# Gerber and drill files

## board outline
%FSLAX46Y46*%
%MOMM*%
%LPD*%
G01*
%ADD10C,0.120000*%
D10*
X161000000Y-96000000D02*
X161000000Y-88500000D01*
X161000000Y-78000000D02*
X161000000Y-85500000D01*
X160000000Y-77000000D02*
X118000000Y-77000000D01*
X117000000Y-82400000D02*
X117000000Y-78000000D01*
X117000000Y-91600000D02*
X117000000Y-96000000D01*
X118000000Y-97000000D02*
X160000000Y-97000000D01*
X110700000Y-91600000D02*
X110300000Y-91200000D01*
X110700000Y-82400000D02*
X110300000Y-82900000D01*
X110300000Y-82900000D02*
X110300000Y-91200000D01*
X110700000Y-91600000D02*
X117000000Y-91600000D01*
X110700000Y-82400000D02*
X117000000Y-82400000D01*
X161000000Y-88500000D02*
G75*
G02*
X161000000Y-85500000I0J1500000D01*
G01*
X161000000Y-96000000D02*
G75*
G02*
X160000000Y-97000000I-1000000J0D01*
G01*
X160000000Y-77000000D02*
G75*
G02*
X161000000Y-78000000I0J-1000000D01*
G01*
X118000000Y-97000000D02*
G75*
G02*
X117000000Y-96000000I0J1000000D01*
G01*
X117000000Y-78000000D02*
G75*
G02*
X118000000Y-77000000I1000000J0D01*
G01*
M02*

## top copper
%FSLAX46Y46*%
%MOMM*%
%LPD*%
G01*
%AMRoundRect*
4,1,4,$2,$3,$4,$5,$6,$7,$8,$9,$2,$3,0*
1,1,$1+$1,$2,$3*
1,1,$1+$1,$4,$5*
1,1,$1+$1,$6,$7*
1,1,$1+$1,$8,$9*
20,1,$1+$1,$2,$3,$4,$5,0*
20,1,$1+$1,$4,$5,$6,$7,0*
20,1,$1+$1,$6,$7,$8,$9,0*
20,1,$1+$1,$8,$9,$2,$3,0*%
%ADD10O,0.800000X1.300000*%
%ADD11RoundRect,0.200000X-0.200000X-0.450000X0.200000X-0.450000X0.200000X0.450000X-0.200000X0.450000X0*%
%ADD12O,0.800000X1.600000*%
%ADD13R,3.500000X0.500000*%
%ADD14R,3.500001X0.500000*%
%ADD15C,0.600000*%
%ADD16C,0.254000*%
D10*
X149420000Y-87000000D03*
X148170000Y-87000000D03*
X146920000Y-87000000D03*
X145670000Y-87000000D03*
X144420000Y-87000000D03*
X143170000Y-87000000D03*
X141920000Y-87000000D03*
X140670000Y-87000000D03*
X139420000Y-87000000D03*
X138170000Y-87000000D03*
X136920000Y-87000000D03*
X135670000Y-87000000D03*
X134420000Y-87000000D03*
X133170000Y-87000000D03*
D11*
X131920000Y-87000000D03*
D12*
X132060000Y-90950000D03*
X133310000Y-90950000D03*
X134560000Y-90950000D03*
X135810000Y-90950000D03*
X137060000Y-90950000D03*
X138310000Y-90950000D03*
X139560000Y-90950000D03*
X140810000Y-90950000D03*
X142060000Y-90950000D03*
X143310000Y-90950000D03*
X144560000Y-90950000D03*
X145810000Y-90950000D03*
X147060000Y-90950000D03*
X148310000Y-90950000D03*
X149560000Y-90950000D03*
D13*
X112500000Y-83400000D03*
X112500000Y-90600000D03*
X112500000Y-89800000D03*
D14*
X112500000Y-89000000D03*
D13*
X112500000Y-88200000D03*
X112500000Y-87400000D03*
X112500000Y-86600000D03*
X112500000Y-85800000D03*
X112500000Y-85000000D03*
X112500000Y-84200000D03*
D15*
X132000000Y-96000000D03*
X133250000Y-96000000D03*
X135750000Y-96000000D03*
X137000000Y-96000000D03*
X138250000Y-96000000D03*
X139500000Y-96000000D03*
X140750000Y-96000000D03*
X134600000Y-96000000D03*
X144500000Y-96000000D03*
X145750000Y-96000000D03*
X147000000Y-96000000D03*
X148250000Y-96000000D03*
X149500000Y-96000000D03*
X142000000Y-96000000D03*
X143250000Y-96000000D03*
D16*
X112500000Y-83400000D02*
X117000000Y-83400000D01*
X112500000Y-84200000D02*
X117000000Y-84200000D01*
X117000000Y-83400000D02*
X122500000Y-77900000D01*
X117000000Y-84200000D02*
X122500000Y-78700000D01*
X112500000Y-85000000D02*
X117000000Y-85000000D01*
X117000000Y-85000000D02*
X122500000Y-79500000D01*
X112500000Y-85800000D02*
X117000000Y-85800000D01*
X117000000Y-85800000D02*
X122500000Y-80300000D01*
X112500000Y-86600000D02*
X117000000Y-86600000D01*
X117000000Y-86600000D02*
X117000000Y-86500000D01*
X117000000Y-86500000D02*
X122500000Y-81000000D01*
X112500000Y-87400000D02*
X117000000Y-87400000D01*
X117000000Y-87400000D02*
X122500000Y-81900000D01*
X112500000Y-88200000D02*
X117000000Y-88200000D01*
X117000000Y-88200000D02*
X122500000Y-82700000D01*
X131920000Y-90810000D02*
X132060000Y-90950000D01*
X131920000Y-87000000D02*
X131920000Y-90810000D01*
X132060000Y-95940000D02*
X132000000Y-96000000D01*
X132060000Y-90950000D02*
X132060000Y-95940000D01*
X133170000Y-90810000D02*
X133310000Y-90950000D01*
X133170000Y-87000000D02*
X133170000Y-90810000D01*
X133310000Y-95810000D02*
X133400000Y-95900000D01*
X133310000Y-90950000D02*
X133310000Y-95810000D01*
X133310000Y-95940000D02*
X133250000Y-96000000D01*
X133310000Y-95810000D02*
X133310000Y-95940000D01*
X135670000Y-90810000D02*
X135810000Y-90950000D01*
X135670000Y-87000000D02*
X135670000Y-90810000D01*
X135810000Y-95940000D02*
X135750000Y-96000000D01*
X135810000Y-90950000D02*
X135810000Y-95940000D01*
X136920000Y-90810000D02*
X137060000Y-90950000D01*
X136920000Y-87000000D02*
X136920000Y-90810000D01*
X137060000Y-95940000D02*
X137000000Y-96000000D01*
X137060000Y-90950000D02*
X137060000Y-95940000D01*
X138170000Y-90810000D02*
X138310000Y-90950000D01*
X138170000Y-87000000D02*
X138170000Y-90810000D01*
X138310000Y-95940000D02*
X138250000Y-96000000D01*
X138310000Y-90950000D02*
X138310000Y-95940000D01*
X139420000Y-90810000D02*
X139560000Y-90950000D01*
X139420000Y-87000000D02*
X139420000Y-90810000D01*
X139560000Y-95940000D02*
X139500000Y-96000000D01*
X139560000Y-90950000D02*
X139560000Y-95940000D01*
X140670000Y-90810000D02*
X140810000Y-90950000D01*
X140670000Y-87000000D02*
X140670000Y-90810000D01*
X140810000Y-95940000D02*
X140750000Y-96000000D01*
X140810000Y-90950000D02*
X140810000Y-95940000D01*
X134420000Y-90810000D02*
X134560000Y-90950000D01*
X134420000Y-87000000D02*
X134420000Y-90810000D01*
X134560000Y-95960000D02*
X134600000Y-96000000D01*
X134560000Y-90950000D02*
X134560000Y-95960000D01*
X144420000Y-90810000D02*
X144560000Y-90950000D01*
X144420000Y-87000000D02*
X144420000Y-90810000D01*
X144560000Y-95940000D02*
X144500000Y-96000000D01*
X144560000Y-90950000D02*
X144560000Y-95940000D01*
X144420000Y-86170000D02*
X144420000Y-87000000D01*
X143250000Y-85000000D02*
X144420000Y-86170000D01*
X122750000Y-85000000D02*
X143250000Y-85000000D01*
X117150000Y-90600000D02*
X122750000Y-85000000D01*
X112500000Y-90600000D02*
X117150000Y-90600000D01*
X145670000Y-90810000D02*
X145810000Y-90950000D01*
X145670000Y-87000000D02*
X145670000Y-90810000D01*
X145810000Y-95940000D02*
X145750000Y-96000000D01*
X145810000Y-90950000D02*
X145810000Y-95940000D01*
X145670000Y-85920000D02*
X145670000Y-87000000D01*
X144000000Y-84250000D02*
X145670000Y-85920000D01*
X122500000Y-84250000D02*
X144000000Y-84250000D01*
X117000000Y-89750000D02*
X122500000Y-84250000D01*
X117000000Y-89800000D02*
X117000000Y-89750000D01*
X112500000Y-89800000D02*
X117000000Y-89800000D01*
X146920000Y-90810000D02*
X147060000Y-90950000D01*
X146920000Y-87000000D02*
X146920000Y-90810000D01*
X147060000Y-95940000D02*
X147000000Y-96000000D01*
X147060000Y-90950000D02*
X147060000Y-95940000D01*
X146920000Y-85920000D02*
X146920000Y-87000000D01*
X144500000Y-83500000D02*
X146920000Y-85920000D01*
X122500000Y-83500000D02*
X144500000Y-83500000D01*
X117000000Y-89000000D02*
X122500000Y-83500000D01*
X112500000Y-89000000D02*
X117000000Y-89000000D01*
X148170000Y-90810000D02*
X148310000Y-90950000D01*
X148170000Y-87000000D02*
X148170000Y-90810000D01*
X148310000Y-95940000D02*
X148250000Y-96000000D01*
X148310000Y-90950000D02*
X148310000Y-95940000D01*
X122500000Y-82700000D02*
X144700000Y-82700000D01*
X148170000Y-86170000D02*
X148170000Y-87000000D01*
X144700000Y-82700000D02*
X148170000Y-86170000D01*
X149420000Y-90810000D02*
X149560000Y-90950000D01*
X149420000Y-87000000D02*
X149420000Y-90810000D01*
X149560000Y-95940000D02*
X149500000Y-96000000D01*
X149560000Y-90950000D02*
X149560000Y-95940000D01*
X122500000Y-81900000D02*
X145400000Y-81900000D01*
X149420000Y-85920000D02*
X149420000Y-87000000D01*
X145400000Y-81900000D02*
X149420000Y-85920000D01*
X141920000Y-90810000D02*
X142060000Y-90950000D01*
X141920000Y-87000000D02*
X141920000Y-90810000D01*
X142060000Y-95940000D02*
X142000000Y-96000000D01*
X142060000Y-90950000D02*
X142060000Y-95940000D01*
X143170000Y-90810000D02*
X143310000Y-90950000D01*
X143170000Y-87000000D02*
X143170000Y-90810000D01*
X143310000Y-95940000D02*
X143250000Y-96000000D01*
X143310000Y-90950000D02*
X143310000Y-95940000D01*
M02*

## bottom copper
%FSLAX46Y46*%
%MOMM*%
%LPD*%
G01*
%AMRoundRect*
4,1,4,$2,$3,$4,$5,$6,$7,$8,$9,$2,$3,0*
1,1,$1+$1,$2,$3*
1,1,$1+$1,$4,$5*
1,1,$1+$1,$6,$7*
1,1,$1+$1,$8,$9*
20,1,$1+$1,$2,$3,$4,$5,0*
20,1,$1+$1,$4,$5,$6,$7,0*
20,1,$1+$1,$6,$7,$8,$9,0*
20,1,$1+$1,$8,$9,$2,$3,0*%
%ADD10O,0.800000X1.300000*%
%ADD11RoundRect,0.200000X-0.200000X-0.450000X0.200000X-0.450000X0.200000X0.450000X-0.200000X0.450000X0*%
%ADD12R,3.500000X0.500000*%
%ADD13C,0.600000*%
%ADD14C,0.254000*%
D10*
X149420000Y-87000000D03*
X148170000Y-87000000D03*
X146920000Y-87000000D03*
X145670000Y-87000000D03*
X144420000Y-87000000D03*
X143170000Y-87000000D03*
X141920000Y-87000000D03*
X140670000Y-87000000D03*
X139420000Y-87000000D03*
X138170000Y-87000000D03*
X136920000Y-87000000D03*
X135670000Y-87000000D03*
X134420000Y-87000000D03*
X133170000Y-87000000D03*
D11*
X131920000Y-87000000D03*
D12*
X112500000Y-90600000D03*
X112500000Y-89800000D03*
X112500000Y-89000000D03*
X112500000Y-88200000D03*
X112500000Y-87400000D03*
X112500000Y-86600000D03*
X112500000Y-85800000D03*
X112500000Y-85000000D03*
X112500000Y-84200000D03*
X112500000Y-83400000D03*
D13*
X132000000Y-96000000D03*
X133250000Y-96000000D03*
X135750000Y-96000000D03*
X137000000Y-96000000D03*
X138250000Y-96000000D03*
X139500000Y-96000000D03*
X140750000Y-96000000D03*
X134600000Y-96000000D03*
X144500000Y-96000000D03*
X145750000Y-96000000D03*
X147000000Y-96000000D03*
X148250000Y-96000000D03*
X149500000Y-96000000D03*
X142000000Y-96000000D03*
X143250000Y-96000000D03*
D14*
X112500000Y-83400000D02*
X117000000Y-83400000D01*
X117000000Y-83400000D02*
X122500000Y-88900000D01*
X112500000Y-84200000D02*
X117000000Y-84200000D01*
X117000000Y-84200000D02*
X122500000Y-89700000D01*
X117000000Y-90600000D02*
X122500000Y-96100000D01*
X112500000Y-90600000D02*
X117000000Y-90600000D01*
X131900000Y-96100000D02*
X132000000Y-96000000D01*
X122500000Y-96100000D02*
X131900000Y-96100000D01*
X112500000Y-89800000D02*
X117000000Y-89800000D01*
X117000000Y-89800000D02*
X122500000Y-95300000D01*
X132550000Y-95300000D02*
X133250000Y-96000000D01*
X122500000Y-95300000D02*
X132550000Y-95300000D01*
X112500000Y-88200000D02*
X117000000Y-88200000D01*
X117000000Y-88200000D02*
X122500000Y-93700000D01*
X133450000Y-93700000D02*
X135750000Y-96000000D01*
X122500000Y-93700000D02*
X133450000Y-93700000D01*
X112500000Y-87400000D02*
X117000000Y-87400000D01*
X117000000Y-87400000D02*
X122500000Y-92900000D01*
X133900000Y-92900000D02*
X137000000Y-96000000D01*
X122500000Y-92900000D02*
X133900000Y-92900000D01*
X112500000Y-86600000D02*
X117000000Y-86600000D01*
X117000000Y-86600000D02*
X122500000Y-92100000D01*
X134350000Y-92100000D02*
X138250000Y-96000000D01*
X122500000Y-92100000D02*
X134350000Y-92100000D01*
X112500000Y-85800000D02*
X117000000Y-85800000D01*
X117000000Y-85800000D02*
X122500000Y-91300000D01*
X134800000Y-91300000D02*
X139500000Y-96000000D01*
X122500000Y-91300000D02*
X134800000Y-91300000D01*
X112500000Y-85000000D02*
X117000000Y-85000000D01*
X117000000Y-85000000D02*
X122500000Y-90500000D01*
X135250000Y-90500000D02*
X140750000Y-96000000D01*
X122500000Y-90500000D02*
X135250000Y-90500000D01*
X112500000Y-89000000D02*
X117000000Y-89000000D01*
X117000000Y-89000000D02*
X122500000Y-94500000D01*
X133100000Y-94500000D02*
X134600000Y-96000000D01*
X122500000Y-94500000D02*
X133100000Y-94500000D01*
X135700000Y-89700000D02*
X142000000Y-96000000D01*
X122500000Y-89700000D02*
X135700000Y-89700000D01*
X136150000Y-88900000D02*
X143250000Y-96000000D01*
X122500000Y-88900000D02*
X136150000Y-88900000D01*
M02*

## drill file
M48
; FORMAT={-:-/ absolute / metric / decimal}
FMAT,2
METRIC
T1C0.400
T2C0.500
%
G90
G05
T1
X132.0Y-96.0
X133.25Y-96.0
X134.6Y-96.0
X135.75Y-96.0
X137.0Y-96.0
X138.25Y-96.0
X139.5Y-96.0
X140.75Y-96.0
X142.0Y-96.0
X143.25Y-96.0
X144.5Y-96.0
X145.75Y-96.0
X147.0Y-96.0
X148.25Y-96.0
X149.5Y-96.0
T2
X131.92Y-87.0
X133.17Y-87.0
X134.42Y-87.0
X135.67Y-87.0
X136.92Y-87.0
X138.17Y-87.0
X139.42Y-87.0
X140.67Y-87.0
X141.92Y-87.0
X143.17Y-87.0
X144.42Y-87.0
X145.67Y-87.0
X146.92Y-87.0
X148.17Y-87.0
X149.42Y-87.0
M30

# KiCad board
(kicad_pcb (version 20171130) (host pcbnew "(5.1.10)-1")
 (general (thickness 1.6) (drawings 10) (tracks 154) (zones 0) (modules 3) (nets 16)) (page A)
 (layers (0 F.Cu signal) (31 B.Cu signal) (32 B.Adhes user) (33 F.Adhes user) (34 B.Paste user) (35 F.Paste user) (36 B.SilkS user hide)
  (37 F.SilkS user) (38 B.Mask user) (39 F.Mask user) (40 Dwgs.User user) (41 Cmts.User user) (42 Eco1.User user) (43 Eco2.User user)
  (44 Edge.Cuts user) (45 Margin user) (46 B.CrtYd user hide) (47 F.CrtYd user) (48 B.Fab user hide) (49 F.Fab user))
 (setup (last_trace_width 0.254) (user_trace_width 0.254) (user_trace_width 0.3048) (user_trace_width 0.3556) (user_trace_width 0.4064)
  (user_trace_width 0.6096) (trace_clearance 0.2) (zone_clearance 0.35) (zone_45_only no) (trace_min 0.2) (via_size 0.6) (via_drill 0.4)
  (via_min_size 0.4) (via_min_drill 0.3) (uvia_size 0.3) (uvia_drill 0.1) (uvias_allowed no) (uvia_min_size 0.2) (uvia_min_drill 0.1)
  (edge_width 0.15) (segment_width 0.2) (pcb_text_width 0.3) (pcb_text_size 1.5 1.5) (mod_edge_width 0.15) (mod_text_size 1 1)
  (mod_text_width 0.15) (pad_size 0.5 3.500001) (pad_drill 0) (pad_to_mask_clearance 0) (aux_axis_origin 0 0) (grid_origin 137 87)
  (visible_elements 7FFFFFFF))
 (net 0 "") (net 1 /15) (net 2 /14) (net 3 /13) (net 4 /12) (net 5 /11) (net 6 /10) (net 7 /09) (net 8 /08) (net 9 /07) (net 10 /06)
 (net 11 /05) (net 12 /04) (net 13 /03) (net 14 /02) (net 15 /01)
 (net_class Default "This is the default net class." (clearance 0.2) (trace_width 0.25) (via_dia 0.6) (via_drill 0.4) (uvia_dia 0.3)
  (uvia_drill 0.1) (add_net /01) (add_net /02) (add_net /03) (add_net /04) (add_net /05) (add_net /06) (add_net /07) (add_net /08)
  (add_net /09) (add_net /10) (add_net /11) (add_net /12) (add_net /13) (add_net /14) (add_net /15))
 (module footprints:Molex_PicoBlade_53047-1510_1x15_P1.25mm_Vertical (layer F.Cu) (at 131.92 87)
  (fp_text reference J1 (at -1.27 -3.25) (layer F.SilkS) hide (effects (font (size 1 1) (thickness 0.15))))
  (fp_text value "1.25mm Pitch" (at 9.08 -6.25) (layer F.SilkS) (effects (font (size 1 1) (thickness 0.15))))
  (pad 15 thru_hole oval (at 17.5 0) (size 0.8 1.3) (drill 0.5) (layers *.Cu *.Mask) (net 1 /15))
  (pad 14 thru_hole oval (at 16.25 0) (size 0.8 1.3) (drill 0.5) (layers *.Cu *.Mask) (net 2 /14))
  (pad 13 thru_hole oval (at 15 0) (size 0.8 1.3) (drill 0.5) (layers *.Cu *.Mask) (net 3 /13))
  (pad 12 thru_hole oval (at 13.75 0) (size 0.8 1.3) (drill 0.5) (layers *.Cu *.Mask) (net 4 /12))
  (pad 11 thru_hole oval (at 12.5 0) (size 0.8 1.3) (drill 0.5) (layers *.Cu *.Mask) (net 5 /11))
  (pad 10 thru_hole oval (at 11.25 0) (size 0.8 1.3) (drill 0.5) (layers *.Cu *.Mask) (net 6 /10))
  (pad 9 thru_hole oval (at 10 0) (size 0.8 1.3) (drill 0.5) (layers *.Cu *.Mask) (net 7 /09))
  (pad 8 thru_hole oval (at 8.75 0) (size 0.8 1.3) (drill 0.5) (layers *.Cu *.Mask) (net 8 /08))
  (pad 7 thru_hole oval (at 7.5 0) (size 0.8 1.3) (drill 0.5) (layers *.Cu *.Mask) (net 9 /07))
  (pad 6 thru_hole oval (at 6.25 0) (size 0.8 1.3) (drill 0.5) (layers *.Cu *.Mask) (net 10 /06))
  (pad 5 thru_hole oval (at 5 0) (size 0.8 1.3) (drill 0.5) (layers *.Cu *.Mask) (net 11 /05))
  (pad 4 thru_hole oval (at 3.75 0) (size 0.8 1.3) (drill 0.5) (layers *.Cu *.Mask) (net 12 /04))
  (pad 3 thru_hole oval (at 2.5 0) (size 0.8 1.3) (drill 0.5) (layers *.Cu *.Mask) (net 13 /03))
  (pad 2 thru_hole oval (at 1.25 0) (size 0.8 1.3) (drill 0.5) (layers *.Cu *.Mask) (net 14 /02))
  (pad 1 thru_hole roundrect (at 0 0) (size 0.8 1.3) (drill 0.5) (layers *.Cu *.Mask) (roundrect_rratio 0.25) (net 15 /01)))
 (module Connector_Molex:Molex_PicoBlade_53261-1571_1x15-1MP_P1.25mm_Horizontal (layer F.Cu) (at 140.81 93.35)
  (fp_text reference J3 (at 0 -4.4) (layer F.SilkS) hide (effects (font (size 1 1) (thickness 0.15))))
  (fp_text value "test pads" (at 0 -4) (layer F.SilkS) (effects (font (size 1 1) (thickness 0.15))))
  (pad 1 smd oval (at -8.75 -2.4) (size 0.8 1.6) (layers F.Cu F.Paste F.Mask) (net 15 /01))
  (pad 2 smd oval (at -7.5 -2.4) (size 0.8 1.6) (layers F.Cu F.Paste F.Mask) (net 14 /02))
  (pad 3 smd oval (at -6.25 -2.4) (size 0.8 1.6) (layers F.Cu F.Paste F.Mask) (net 13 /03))
  (pad 4 smd oval (at -5 -2.4) (size 0.8 1.6) (layers F.Cu F.Paste F.Mask) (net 12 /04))
  (pad 5 smd oval (at -3.75 -2.4) (size 0.8 1.6) (layers F.Cu F.Paste F.Mask) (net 11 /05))
  (pad 6 smd oval (at -2.5 -2.4) (size 0.8 1.6) (layers F.Cu F.Paste F.Mask) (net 10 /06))
  (pad 7 smd oval (at -1.25 -2.4) (size 0.8 1.6) (layers F.Cu F.Paste F.Mask) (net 9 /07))
  (pad 8 smd oval (at 0 -2.4) (size 0.8 1.6) (layers F.Cu F.Paste F.Mask) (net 8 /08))
  (pad 9 smd oval (at 1.25 -2.4) (size 0.8 1.6) (layers F.Cu F.Paste F.Mask) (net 7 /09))
  (pad 10 smd oval (at 2.5 -2.4) (size 0.8 1.6) (layers F.Cu F.Paste F.Mask) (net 6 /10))
  (pad 11 smd oval (at 3.75 -2.4) (size 0.8 1.6) (layers F.Cu F.Paste F.Mask) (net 5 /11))
  (pad 12 smd oval (at 5 -2.4) (size 0.8 1.6) (layers F.Cu F.Paste F.Mask) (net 4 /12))
  (pad 13 smd oval (at 6.25 -2.4) (size 0.8 1.6) (layers F.Cu F.Paste F.Mask) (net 3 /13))
  (pad 14 smd oval (at 7.5 -2.4) (size 0.8 1.6) (layers F.Cu F.Paste F.Mask) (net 2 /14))
  (pad 15 smd oval (at 8.75 -2.4) (size 0.8 1.6) (layers F.Cu F.Paste F.Mask) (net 1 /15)))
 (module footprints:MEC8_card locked (layer F.Cu) (at 112.5 87 90)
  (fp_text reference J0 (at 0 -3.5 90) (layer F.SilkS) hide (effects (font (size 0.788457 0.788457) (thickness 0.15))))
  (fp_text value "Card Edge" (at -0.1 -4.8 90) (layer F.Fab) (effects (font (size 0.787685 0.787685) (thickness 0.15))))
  (fp_line (start -9 48.5) (end -1.5 48.5) (layer Edge.Cuts) (width 0.12))
  (fp_line (start 9 48.5) (end 1.5 48.5) (layer Edge.Cuts) (width 0.12))
  (fp_line (start 10 47.5) (end 10 5.5) (layer Edge.Cuts) (width 0.12))
  (fp_line (start 4.6 4.5) (end 9 4.5) (layer Edge.Cuts) (width 0.12))
  (fp_line (start -4.6 4.5) (end -9 4.5) (layer Edge.Cuts) (width 0.12))
  (fp_line (start -10 5.5) (end -10 47.5) (layer Edge.Cuts) (width 0.12))
  (fp_line (start -4.6 -1.8) (end -4.2 -2.2) (layer Edge.Cuts) (width 0.12))
  (fp_line (start 4.6 -1.8) (end 4.1 -2.2) (layer Edge.Cuts) (width 0.12))
  (fp_line (start 4.1 -2.2) (end -4.2 -2.2) (layer Edge.Cuts) (width 0.12))
  (fp_line (start -4.6 -1.8) (end -4.6 4.5) (layer Edge.Cuts) (width 0.12))
  (fp_line (start 4.6 -1.8) (end 4.6 4.5) (layer Edge.Cuts) (width 0.12))
  (fp_arc (start 0 48.5) (end 1.5 48.5) (angle -180) (layer Edge.Cuts) (width 0.12))
  (fp_arc (start -9 47.5) (end -10 47.5) (angle -90) (layer Edge.Cuts) (width 0.12))
  (fp_arc (start 9 47.5) (end 9 48.5) (angle -90) (layer Edge.Cuts) (width 0.12))
  (fp_arc (start -9 5.5) (end -9 4.5) (angle -90) (layer Edge.Cuts) (width 0.12))
  (fp_arc (start 9 5.5) (end 10 5.5) (angle -90) (layer Edge.Cuts) (width 0.12))
  (pad 20 smd rect (at 3.6 0 90) (size 0.5 3.5) (layers F.Cu F.Paste F.Mask))
  (pad 11 smd rect (at -3.6 0 90) (size 0.5 3.5) (layers F.Cu F.Paste F.Mask) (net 5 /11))
  (pad 12 smd rect (at -2.8 0 90) (size 0.5 3.5) (layers F.Cu F.Paste F.Mask) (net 4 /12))
  (pad 13 smd rect (at -2 0 90) (size 0.5 3.500001) (layers F.Cu F.Paste F.Mask) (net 3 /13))
  (pad 14 smd rect (at -1.2 0 90) (size 0.5 3.5) (layers F.Cu F.Paste F.Mask) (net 2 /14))
  (pad 15 smd rect (at -0.4 0 90) (size 0.5 3.5) (layers F.Cu F.Paste F.Mask) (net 1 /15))
  (pad 16 smd rect (at 0.4 0 90) (size 0.5 3.5) (layers F.Cu F.Paste F.Mask))
  (pad 17 smd rect (at 1.2 0 90) (size 0.5 3.5) (layers F.Cu F.Paste F.Mask))
  (pad 18 smd rect (at 2 0 90) (size 0.5 3.5) (layers F.Cu F.Paste F.Mask))
  (pad 19 smd rect (at 2.8 0 90) (size 0.5 3.5) (layers F.Cu F.Paste F.Mask))
  (pad 1 smd rect (at -3.6 0 90) (size 0.5 3.5) (layers B.Cu B.Paste B.Mask) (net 15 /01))
  (pad 2 smd rect (at -2.8 0 90) (size 0.5 3.5) (layers B.Cu B.Paste B.Mask) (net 14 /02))
  (pad 3 smd rect (at -2 0 90) (size 0.5 3.5) (layers B.Cu B.Paste B.Mask) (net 13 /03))
  (pad 4 smd rect (at -1.2 0 90) (size 0.5 3.5) (layers B.Cu B.Paste B.Mask) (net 12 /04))
  (pad 5 smd rect (at -0.4 0 90) (size 0.5 3.5) (layers B.Cu B.Paste B.Mask) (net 11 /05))
  (pad 6 smd rect (at 0.4 0 90) (size 0.5 3.5) (layers B.Cu B.Paste B.Mask) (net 10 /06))
  (pad 7 smd rect (at 1.2 0 90) (size 0.5 3.5) (layers B.Cu B.Paste B.Mask) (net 9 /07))
  (pad 8 smd rect (at 2 0 90) (size 0.5 3.5) (layers B.Cu B.Paste B.Mask) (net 8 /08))
  (pad 9 smd rect (at 2.8 0 90) (size 0.5 3.5) (layers B.Cu B.Paste B.Mask) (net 7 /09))
  (pad 10 smd rect (at 3.6 0 90) (size 0.5 3.5) (layers B.Cu B.Paste B.Mask) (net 6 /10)))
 (segment (start 112.5 83.4) (end 117 83.4) (width 0.254) (layer F.Cu) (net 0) (status 10))
 (segment (start 112.5 84.2) (end 117 84.2) (width 0.254) (layer F.Cu) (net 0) (status 10))
 (segment (start 117 83.4) (end 122.5 77.9) (width 0.254) (layer F.Cu) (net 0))
 (segment (start 117 84.2) (end 122.5 78.7) (width 0.254) (layer F.Cu) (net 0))
 (segment (start 112.5 83.4) (end 117 83.4) (width 0.254) (layer B.Cu) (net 6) (status 10))
 (segment (start 117 83.4) (end 122.5 88.9) (width 0.254) (layer B.Cu) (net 6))
 (segment (start 112.5 85) (end 117 85) (width 0.254) (layer F.Cu) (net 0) (status 10))
 (segment (start 117 85) (end 122.5 79.5) (width 0.254) (layer F.Cu) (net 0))
 (segment (start 112.5 85.8) (end 117 85.8) (width 0.254) (layer F.Cu) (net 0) (status 10))
 (segment (start 117 85.8) (end 122.5 80.3) (width 0.254) (layer F.Cu) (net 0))
 (segment (start 112.5 86.6) (end 117 86.6) (width 0.254) (layer F.Cu) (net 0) (status 10))
 (segment (start 117 86.6) (end 117 86.5) (width 0.254) (layer F.Cu) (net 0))
 (segment (start 117 86.5) (end 122.5 81) (width 0.254) (layer F.Cu) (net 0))
 (segment (start 112.5 87.4) (end 117 87.4) (width 0.254) (layer F.Cu) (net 1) (status 10))
 (segment (start 117 87.4) (end 122.5 81.9) (width 0.254) (layer F.Cu) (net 1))
 (segment (start 112.5 88.2) (end 117 88.2) (width 0.254) (layer F.Cu) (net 2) (status 10))
 (segment (start 117 88.2) (end 122.5 82.7) (width 0.254) (layer F.Cu) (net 2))
 (segment (start 112.5 84.2) (end 117 84.2) (width 0.254) (layer B.Cu) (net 7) (status 10))
 (segment (start 117 84.2) (end 122.5 89.7) (width 0.254) (layer B.Cu) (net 7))
 (segment (start 117 90.6) (end 122.5 96.1) (width 0.254) (layer B.Cu) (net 15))
 (segment (start 112.5 90.6) (end 117 90.6) (width 0.254) (layer B.Cu) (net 15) (status 10))
 (segment (start 131.92 90.81) (end 132.06 90.95) (width 0.254) (layer F.Cu) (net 15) (status 30))
 (segment (start 131.92 87) (end 131.92 90.81) (width 0.254) (layer F.Cu) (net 15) (status 30))
 (via (at 132 96) (size 0.6) (drill 0.4) (layers F.Cu B.Cu) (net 15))
 (segment (start 132.06 95.94) (end 132 96) (width 0.254) (layer F.Cu) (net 15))
 (segment (start 132.06 90.95) (end 132.06 95.94) (width 0.254) (layer F.Cu) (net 15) (status 10))
 (segment (start 131.9 96.1) (end 132 96) (width 0.254) (layer B.Cu) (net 15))
 (segment (start 122.5 96.1) (end 131.9 96.1) (width 0.254) (layer B.Cu) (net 15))
 (segment (start 112.5 89.8) (end 117 89.8) (width 0.254) (layer B.Cu) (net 14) (status 10))
 (segment (start 117 89.8) (end 122.5 95.3) (width 0.254) (layer B.Cu) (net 14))
 (segment (start 133.17 90.81) (end 133.31 90.95) (width 0.254) (layer F.Cu) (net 14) (status 30))
 (segment (start 133.17 87) (end 133.17 90.81) (width 0.254) (layer F.Cu) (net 14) (status 30))
 (segment (start 133.31 95.81) (end 133.4 95.9) (width 0.254) (layer F.Cu) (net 14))
 (segment (start 133.31 90.95) (end 133.31 95.81) (width 0.254) (layer F.Cu) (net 14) (status 10))
 (via (at 133.25 96) (size 0.6) (drill 0.4) (layers F.Cu B.Cu) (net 14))
 (segment (start 133.31 95.94) (end 133.25 96) (width 0.254) (layer F.Cu) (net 14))
 (segment (start 133.31 95.81) (end 133.31 95.94) (width 0.254) (layer F.Cu) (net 14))
 (segment (start 132.55 95.3) (end 133.25 96) (width 0.254) (layer B.Cu) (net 14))
 (segment (start 122.5 95.3) (end 132.55 95.3) (width 0.254) (layer B.Cu) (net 14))
 (segment (start 112.5 88.2) (end 117 88.2) (width 0.254) (layer B.Cu) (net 12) (status 10))
 (segment (start 117 88.2) (end 122.5 93.7) (width 0.254) (layer B.Cu) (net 12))
 (segment (start 135.67 90.81) (end 135.81 90.95) (width 0.254) (layer F.Cu) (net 12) (status 30))
 (segment (start 135.67 87) (end 135.67 90.81) (width 0.254) (layer F.Cu) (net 12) (status 30))
 (via (at 135.75 96) (size 0.6) (drill 0.4) (layers F.Cu B.Cu) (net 12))
 (segment (start 135.81 95.94) (end 135.75 96) (width 0.254) (layer F.Cu) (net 12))
 (segment (start 135.81 90.95) (end 135.81 95.94) (width 0.254) (layer F.Cu) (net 12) (status 10))
 (segment (start 133.45 93.7) (end 135.75 96) (width 0.254) (layer B.Cu) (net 12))
 (segment (start 122.5 93.7) (end 133.45 93.7) (width 0.254) (layer B.Cu) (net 12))
 (segment (start 112.5 87.4) (end 117 87.4) (width 0.254) (layer B.Cu) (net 11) (status 10))
 (segment (start 117 87.4) (end 122.5 92.9) (width 0.254) (layer B.Cu) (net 11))
 (segment (start 136.92 90.81) (end 137.06 90.95) (width 0.254) (layer F.Cu) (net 11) (status 30))
 (segment (start 136.92 87) (end 136.92 90.81) (width 0.254) (layer F.Cu) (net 11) (status 30))
 (via (at 137 96) (size 0.6) (drill 0.4) (layers F.Cu B.Cu) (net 11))
 (segment (start 137.06 95.94) (end 137 96) (width 0.254) (layer F.Cu) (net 11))
 (segment (start 137.06 90.95) (end 137.06 95.94) (width 0.254) (layer F.Cu) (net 11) (status 10))
 (segment (start 133.9 92.9) (end 137 96) (width 0.254) (layer B.Cu) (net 11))
 (segment (start 122.5 92.9) (end 133.9 92.9) (width 0.254) (layer B.Cu) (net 11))
 (segment (start 112.5 86.6) (end 117 86.6) (width 0.254) (layer B.Cu) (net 10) (status 10))
 (segment (start 117 86.6) (end 122.5 92.1) (width 0.254) (layer B.Cu) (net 10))
 (segment (start 138.17 90.81) (end 138.31 90.95) (width 0.254) (layer F.Cu) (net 10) (status 30))
 (segment (start 138.17 87) (end 138.17 90.81) (width 0.254) (layer F.Cu) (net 10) (status 30))
 (via (at 138.25 96) (size 0.6) (drill 0.4) (layers F.Cu B.Cu) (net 10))
 (segment (start 138.31 95.94) (end 138.25 96) (width 0.254) (layer F.Cu) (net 10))
 (segment (start 138.31 90.95) (end 138.31 95.94) (width 0.254) (layer F.Cu) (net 10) (status 10))
 (segment (start 134.35 92.1) (end 138.25 96) (width 0.254) (layer B.Cu) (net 10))
 (segment (start 122.5 92.1) (end 134.35 92.1) (width 0.254) (layer B.Cu) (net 10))
 (segment (start 112.5 85.8) (end 117 85.8) (width 0.254) (layer B.Cu) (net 9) (status 10))
 (segment (start 117 85.8) (end 122.5 91.3) (width 0.254) (layer B.Cu) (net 9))
 (segment (start 139.42 90.81) (end 139.56 90.95) (width 0.254) (layer F.Cu) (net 9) (status 30))
 (segment (start 139.42 87) (end 139.42 90.81) (width 0.254) (layer F.Cu) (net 9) (status 30))
 (via (at 139.5 96) (size 0.6) (drill 0.4) (layers F.Cu B.Cu) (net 9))
 (segment (start 139.56 95.94) (end 139.5 96) (width 0.254) (layer F.Cu) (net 9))
 (segment (start 139.56 90.95) (end 139.56 95.94) (width 0.254) (layer F.Cu) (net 9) (status 10))
 (segment (start 134.8 91.3) (end 139.5 96) (width 0.254) (layer B.Cu) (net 9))
 (segment (start 122.5 91.3) (end 134.8 91.3) (width 0.254) (layer B.Cu) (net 9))
 (segment (start 112.5 85) (end 117 85) (width 0.254) (layer B.Cu) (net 8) (status 10))
 (segment (start 117 85) (end 122.5 90.5) (width 0.254) (layer B.Cu) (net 8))
 (segment (start 140.67 90.81) (end 140.81 90.95) (width 0.254) (layer F.Cu) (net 8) (status 30))
 (segment (start 140.67 87) (end 140.67 90.81) (width 0.254) (layer F.Cu) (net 8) (status 30))
 (via (at 140.75 96) (size 0.6) (drill 0.4) (layers F.Cu B.Cu) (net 8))
 (segment (start 140.81 95.94) (end 140.75 96) (width 0.254) (layer F.Cu) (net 8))
 (segment (start 140.81 90.95) (end 140.81 95.94) (width 0.254) (layer F.Cu) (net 8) (status 10))
 (segment (start 135.25 90.5) (end 140.75 96) (width 0.254) (layer B.Cu) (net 8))
 (segment (start 122.5 90.5) (end 135.25 90.5) (width 0.254) (layer B.Cu) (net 8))
 (segment (start 112.5 89) (end 117 89) (width 0.254) (layer B.Cu) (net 13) (status 10))
 (segment (start 117 89) (end 122.5 94.5) (width 0.254) (layer B.Cu) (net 13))
 (segment (start 134.42 90.81) (end 134.56 90.95) (width 0.254) (layer F.Cu) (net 13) (status 30))
 (segment (start 134.42 87) (end 134.42 90.81) (width 0.254) (layer F.Cu) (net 13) (status 30))
 (via (at 134.6 96) (size 0.6) (drill 0.4) (layers F.Cu B.Cu) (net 13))
 (segment (start 134.56 95.96) (end 134.6 96) (width 0.254) (layer F.Cu) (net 13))
 (segment (start 134.56 90.95) (end 134.56 95.96) (width 0.254) (layer F.Cu) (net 13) (status 10))
 (segment (start 133.1 94.5) (end 134.6 96) (width 0.254) (layer B.Cu) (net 13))
 (segment (start 122.5 94.5) (end 133.1 94.5) (width 0.254) (layer B.Cu) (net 13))
 (segment (start 144.42 90.81) (end 144.56 90.95) (width 0.254) (layer F.Cu) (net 5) (status 30))
 (segment (start 144.42 87) (end 144.42 90.81) (width 0.254) (layer F.Cu) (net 5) (status 30))
 (via (at 144.5 96) (size 0.6) (drill 0.4) (layers F.Cu B.Cu) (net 5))
 (segment (start 144.56 95.94) (end 144.5 96) (width 0.254) (layer F.Cu) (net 5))
 (segment (start 144.56 90.95) (end 144.56 95.94) (width 0.254) (layer F.Cu) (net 5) (status 10))
 (segment (start 144.42 86.17) (end 144.42 87) (width 0.254) (layer F.Cu) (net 5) (status 20))
 (segment (start 143.25 85) (end 144.42 86.17) (width 0.254) (layer F.Cu) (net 5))
 (segment (start 122.75 85) (end 143.25 85) (width 0.254) (layer F.Cu) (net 5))
 (segment (start 117.15 90.6) (end 122.75 85) (width 0.254) (layer F.Cu) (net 5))
 (segment (start 112.5 90.6) (end 117.15 90.6) (width 0.254) (layer F.Cu) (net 5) (status 10))
 (segment (start 145.67 90.81) (end 145.81 90.95) (width 0.254) (layer F.Cu) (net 4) (status 30))
 (segment (start 145.67 87) (end 145.67 90.81) (width 0.254) (layer F.Cu) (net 4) (status 30))
 (via (at 145.75 96) (size 0.6) (drill 0.4) (layers F.Cu B.Cu) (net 4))
 (segment (start 145.81 95.94) (end 145.75 96) (width 0.254) (layer F.Cu) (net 4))
 (segment (start 145.81 90.95) (end 145.81 95.94) (width 0.254) (layer F.Cu) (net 4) (status 10))
 (segment (start 145.67 85.92) (end 145.67 87) (width 0.254) (layer F.Cu) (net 4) (status 20))
 (segment (start 144 84.25) (end 145.67 85.92) (width 0.254) (layer F.Cu) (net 4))
 (segment (start 122.5 84.25) (end 144 84.25) (width 0.254) (layer F.Cu) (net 4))
 (segment (start 117 89.75) (end 122.5 84.25) (width 0.254) (layer F.Cu) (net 4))
 (segment (start 117 89.8) (end 117 89.75) (width 0.254) (layer F.Cu) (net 4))
 (segment (start 112.5 89.8) (end 117 89.8) (width 0.254) (layer F.Cu) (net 4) (status 10))
 (segment (start 146.92 90.81) (end 147.06 90.95) (width 0.254) (layer F.Cu) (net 3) (status 30))
 (segment (start 146.92 87) (end 146.92 90.81) (width 0.254) (layer F.Cu) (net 3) (status 30))
 (via (at 147 96) (size 0.6) (drill 0.4) (layers F.Cu B.Cu) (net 3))
 (segment (start 147.06 95.94) (end 147 96) (width 0.254) (layer F.Cu) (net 3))
 (segment (start 147.06 90.95) (end 147.06 95.94) (width 0.254) (layer F.Cu) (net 3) (status 10))
 (segment (start 146.92 85.92) (end 146.92 87) (width 0.254) (layer F.Cu) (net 3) (status 20))
 (segment (start 144.5 83.5) (end 146.92 85.92) (width 0.254) (layer F.Cu) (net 3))
 (segment (start 122.5 83.5) (end 144.5 83.5) (width 0.254) (layer F.Cu) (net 3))
 (segment (start 117 89) (end 122.5 83.5) (width 0.254) (layer F.Cu) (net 3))
 (segment (start 112.5 89) (end 117 89) (width 0.254) (layer F.Cu) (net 3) (status 10))
 (segment (start 148.17 90.81) (end 148.31 90.95) (width 0.254) (layer F.Cu) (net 2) (status 30))
 (segment (start 148.17 87) (end 148.17 90.81) (width 0.254) (layer F.Cu) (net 2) (status 30))
 (via (at 148.25 96) (size 0.6) (drill 0.4) (layers F.Cu B.Cu) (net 2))
 (segment (start 148.31 95.94) (end 148.25 96) (width 0.254) (layer F.Cu) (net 2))
 (segment (start 148.31 90.95) (end 148.31 95.94) (width 0.254) (layer F.Cu) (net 2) (status 10))
 (segment (start 122.5 82.7) (end 144.7 82.7) (width 0.254) (layer F.Cu) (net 2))
 (segment (start 148.17 86.17) (end 148.17 87) (width 0.254) (layer F.Cu) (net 2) (status 20))
 (segment (start 144.7 82.7) (end 148.17 86.17) (width 0.254) (layer F.Cu) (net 2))
 (segment (start 149.42 90.81) (end 149.56 90.95) (width 0.254) (layer F.Cu) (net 1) (status 30))
 (segment (start 149.42 87) (end 149.42 90.81) (width 0.254) (layer F.Cu) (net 1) (status 30))
 (via (at 149.5 96) (size 0.6) (drill 0.4) (layers F.Cu B.Cu) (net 1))
 (segment (start 149.56 95.94) (end 149.5 96) (width 0.254) (layer F.Cu) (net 1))
 (segment (start 149.56 90.95) (end 149.56 95.94) (width 0.254) (layer F.Cu) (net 1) (status 10))
 (segment (start 122.5 81.9) (end 145.4 81.9) (width 0.254) (layer F.Cu) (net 1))
 (segment (start 149.42 85.92) (end 149.42 87) (width 0.254) (layer F.Cu) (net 1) (status 20))
 (segment (start 145.4 81.9) (end 149.42 85.92) (width 0.254) (layer F.Cu) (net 1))
 (segment (start 141.92 90.81) (end 142.06 90.95) (width 0.254) (layer F.Cu) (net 7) (status 30))
 (segment (start 141.92 87) (end 141.92 90.81) (width 0.254) (layer F.Cu) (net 7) (status 30))
 (via (at 142 96) (size 0.6) (drill 0.4) (layers F.Cu B.Cu) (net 7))
 (segment (start 142.06 95.94) (end 142 96) (width 0.254) (layer F.Cu) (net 7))
 (segment (start 142.06 90.95) (end 142.06 95.94) (width 0.254) (layer F.Cu) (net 7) (status 10))
 (segment (start 135.7 89.7) (end 142 96) (width 0.254) (layer B.Cu) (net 7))
 (segment (start 122.5 89.7) (end 135.7 89.7) (width 0.254) (layer B.Cu) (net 7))
 (segment (start 143.17 90.81) (end 143.31 90.95) (width 0.254) (layer F.Cu) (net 6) (status 30))
 (segment (start 143.17 87) (end 143.17 90.81) (width 0.254) (layer F.Cu) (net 6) (status 30))
 (via (at 143.25 96) (size 0.6) (drill 0.4) (layers F.Cu B.Cu) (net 6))
 (segment (start 143.31 95.94) (end 143.25 96) (width 0.254) (layer F.Cu) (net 6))
 (segment (start 143.31 90.95) (end 143.31 95.94) (width 0.254) (layer F.Cu) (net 6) (status 10))
 (segment (start 136.15 88.9) (end 143.25 96) (width 0.254) (layer B.Cu) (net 6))
 (segment (start 122.5 88.9) (end 136.15 88.9) (width 0.254) (layer B.Cu) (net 6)))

